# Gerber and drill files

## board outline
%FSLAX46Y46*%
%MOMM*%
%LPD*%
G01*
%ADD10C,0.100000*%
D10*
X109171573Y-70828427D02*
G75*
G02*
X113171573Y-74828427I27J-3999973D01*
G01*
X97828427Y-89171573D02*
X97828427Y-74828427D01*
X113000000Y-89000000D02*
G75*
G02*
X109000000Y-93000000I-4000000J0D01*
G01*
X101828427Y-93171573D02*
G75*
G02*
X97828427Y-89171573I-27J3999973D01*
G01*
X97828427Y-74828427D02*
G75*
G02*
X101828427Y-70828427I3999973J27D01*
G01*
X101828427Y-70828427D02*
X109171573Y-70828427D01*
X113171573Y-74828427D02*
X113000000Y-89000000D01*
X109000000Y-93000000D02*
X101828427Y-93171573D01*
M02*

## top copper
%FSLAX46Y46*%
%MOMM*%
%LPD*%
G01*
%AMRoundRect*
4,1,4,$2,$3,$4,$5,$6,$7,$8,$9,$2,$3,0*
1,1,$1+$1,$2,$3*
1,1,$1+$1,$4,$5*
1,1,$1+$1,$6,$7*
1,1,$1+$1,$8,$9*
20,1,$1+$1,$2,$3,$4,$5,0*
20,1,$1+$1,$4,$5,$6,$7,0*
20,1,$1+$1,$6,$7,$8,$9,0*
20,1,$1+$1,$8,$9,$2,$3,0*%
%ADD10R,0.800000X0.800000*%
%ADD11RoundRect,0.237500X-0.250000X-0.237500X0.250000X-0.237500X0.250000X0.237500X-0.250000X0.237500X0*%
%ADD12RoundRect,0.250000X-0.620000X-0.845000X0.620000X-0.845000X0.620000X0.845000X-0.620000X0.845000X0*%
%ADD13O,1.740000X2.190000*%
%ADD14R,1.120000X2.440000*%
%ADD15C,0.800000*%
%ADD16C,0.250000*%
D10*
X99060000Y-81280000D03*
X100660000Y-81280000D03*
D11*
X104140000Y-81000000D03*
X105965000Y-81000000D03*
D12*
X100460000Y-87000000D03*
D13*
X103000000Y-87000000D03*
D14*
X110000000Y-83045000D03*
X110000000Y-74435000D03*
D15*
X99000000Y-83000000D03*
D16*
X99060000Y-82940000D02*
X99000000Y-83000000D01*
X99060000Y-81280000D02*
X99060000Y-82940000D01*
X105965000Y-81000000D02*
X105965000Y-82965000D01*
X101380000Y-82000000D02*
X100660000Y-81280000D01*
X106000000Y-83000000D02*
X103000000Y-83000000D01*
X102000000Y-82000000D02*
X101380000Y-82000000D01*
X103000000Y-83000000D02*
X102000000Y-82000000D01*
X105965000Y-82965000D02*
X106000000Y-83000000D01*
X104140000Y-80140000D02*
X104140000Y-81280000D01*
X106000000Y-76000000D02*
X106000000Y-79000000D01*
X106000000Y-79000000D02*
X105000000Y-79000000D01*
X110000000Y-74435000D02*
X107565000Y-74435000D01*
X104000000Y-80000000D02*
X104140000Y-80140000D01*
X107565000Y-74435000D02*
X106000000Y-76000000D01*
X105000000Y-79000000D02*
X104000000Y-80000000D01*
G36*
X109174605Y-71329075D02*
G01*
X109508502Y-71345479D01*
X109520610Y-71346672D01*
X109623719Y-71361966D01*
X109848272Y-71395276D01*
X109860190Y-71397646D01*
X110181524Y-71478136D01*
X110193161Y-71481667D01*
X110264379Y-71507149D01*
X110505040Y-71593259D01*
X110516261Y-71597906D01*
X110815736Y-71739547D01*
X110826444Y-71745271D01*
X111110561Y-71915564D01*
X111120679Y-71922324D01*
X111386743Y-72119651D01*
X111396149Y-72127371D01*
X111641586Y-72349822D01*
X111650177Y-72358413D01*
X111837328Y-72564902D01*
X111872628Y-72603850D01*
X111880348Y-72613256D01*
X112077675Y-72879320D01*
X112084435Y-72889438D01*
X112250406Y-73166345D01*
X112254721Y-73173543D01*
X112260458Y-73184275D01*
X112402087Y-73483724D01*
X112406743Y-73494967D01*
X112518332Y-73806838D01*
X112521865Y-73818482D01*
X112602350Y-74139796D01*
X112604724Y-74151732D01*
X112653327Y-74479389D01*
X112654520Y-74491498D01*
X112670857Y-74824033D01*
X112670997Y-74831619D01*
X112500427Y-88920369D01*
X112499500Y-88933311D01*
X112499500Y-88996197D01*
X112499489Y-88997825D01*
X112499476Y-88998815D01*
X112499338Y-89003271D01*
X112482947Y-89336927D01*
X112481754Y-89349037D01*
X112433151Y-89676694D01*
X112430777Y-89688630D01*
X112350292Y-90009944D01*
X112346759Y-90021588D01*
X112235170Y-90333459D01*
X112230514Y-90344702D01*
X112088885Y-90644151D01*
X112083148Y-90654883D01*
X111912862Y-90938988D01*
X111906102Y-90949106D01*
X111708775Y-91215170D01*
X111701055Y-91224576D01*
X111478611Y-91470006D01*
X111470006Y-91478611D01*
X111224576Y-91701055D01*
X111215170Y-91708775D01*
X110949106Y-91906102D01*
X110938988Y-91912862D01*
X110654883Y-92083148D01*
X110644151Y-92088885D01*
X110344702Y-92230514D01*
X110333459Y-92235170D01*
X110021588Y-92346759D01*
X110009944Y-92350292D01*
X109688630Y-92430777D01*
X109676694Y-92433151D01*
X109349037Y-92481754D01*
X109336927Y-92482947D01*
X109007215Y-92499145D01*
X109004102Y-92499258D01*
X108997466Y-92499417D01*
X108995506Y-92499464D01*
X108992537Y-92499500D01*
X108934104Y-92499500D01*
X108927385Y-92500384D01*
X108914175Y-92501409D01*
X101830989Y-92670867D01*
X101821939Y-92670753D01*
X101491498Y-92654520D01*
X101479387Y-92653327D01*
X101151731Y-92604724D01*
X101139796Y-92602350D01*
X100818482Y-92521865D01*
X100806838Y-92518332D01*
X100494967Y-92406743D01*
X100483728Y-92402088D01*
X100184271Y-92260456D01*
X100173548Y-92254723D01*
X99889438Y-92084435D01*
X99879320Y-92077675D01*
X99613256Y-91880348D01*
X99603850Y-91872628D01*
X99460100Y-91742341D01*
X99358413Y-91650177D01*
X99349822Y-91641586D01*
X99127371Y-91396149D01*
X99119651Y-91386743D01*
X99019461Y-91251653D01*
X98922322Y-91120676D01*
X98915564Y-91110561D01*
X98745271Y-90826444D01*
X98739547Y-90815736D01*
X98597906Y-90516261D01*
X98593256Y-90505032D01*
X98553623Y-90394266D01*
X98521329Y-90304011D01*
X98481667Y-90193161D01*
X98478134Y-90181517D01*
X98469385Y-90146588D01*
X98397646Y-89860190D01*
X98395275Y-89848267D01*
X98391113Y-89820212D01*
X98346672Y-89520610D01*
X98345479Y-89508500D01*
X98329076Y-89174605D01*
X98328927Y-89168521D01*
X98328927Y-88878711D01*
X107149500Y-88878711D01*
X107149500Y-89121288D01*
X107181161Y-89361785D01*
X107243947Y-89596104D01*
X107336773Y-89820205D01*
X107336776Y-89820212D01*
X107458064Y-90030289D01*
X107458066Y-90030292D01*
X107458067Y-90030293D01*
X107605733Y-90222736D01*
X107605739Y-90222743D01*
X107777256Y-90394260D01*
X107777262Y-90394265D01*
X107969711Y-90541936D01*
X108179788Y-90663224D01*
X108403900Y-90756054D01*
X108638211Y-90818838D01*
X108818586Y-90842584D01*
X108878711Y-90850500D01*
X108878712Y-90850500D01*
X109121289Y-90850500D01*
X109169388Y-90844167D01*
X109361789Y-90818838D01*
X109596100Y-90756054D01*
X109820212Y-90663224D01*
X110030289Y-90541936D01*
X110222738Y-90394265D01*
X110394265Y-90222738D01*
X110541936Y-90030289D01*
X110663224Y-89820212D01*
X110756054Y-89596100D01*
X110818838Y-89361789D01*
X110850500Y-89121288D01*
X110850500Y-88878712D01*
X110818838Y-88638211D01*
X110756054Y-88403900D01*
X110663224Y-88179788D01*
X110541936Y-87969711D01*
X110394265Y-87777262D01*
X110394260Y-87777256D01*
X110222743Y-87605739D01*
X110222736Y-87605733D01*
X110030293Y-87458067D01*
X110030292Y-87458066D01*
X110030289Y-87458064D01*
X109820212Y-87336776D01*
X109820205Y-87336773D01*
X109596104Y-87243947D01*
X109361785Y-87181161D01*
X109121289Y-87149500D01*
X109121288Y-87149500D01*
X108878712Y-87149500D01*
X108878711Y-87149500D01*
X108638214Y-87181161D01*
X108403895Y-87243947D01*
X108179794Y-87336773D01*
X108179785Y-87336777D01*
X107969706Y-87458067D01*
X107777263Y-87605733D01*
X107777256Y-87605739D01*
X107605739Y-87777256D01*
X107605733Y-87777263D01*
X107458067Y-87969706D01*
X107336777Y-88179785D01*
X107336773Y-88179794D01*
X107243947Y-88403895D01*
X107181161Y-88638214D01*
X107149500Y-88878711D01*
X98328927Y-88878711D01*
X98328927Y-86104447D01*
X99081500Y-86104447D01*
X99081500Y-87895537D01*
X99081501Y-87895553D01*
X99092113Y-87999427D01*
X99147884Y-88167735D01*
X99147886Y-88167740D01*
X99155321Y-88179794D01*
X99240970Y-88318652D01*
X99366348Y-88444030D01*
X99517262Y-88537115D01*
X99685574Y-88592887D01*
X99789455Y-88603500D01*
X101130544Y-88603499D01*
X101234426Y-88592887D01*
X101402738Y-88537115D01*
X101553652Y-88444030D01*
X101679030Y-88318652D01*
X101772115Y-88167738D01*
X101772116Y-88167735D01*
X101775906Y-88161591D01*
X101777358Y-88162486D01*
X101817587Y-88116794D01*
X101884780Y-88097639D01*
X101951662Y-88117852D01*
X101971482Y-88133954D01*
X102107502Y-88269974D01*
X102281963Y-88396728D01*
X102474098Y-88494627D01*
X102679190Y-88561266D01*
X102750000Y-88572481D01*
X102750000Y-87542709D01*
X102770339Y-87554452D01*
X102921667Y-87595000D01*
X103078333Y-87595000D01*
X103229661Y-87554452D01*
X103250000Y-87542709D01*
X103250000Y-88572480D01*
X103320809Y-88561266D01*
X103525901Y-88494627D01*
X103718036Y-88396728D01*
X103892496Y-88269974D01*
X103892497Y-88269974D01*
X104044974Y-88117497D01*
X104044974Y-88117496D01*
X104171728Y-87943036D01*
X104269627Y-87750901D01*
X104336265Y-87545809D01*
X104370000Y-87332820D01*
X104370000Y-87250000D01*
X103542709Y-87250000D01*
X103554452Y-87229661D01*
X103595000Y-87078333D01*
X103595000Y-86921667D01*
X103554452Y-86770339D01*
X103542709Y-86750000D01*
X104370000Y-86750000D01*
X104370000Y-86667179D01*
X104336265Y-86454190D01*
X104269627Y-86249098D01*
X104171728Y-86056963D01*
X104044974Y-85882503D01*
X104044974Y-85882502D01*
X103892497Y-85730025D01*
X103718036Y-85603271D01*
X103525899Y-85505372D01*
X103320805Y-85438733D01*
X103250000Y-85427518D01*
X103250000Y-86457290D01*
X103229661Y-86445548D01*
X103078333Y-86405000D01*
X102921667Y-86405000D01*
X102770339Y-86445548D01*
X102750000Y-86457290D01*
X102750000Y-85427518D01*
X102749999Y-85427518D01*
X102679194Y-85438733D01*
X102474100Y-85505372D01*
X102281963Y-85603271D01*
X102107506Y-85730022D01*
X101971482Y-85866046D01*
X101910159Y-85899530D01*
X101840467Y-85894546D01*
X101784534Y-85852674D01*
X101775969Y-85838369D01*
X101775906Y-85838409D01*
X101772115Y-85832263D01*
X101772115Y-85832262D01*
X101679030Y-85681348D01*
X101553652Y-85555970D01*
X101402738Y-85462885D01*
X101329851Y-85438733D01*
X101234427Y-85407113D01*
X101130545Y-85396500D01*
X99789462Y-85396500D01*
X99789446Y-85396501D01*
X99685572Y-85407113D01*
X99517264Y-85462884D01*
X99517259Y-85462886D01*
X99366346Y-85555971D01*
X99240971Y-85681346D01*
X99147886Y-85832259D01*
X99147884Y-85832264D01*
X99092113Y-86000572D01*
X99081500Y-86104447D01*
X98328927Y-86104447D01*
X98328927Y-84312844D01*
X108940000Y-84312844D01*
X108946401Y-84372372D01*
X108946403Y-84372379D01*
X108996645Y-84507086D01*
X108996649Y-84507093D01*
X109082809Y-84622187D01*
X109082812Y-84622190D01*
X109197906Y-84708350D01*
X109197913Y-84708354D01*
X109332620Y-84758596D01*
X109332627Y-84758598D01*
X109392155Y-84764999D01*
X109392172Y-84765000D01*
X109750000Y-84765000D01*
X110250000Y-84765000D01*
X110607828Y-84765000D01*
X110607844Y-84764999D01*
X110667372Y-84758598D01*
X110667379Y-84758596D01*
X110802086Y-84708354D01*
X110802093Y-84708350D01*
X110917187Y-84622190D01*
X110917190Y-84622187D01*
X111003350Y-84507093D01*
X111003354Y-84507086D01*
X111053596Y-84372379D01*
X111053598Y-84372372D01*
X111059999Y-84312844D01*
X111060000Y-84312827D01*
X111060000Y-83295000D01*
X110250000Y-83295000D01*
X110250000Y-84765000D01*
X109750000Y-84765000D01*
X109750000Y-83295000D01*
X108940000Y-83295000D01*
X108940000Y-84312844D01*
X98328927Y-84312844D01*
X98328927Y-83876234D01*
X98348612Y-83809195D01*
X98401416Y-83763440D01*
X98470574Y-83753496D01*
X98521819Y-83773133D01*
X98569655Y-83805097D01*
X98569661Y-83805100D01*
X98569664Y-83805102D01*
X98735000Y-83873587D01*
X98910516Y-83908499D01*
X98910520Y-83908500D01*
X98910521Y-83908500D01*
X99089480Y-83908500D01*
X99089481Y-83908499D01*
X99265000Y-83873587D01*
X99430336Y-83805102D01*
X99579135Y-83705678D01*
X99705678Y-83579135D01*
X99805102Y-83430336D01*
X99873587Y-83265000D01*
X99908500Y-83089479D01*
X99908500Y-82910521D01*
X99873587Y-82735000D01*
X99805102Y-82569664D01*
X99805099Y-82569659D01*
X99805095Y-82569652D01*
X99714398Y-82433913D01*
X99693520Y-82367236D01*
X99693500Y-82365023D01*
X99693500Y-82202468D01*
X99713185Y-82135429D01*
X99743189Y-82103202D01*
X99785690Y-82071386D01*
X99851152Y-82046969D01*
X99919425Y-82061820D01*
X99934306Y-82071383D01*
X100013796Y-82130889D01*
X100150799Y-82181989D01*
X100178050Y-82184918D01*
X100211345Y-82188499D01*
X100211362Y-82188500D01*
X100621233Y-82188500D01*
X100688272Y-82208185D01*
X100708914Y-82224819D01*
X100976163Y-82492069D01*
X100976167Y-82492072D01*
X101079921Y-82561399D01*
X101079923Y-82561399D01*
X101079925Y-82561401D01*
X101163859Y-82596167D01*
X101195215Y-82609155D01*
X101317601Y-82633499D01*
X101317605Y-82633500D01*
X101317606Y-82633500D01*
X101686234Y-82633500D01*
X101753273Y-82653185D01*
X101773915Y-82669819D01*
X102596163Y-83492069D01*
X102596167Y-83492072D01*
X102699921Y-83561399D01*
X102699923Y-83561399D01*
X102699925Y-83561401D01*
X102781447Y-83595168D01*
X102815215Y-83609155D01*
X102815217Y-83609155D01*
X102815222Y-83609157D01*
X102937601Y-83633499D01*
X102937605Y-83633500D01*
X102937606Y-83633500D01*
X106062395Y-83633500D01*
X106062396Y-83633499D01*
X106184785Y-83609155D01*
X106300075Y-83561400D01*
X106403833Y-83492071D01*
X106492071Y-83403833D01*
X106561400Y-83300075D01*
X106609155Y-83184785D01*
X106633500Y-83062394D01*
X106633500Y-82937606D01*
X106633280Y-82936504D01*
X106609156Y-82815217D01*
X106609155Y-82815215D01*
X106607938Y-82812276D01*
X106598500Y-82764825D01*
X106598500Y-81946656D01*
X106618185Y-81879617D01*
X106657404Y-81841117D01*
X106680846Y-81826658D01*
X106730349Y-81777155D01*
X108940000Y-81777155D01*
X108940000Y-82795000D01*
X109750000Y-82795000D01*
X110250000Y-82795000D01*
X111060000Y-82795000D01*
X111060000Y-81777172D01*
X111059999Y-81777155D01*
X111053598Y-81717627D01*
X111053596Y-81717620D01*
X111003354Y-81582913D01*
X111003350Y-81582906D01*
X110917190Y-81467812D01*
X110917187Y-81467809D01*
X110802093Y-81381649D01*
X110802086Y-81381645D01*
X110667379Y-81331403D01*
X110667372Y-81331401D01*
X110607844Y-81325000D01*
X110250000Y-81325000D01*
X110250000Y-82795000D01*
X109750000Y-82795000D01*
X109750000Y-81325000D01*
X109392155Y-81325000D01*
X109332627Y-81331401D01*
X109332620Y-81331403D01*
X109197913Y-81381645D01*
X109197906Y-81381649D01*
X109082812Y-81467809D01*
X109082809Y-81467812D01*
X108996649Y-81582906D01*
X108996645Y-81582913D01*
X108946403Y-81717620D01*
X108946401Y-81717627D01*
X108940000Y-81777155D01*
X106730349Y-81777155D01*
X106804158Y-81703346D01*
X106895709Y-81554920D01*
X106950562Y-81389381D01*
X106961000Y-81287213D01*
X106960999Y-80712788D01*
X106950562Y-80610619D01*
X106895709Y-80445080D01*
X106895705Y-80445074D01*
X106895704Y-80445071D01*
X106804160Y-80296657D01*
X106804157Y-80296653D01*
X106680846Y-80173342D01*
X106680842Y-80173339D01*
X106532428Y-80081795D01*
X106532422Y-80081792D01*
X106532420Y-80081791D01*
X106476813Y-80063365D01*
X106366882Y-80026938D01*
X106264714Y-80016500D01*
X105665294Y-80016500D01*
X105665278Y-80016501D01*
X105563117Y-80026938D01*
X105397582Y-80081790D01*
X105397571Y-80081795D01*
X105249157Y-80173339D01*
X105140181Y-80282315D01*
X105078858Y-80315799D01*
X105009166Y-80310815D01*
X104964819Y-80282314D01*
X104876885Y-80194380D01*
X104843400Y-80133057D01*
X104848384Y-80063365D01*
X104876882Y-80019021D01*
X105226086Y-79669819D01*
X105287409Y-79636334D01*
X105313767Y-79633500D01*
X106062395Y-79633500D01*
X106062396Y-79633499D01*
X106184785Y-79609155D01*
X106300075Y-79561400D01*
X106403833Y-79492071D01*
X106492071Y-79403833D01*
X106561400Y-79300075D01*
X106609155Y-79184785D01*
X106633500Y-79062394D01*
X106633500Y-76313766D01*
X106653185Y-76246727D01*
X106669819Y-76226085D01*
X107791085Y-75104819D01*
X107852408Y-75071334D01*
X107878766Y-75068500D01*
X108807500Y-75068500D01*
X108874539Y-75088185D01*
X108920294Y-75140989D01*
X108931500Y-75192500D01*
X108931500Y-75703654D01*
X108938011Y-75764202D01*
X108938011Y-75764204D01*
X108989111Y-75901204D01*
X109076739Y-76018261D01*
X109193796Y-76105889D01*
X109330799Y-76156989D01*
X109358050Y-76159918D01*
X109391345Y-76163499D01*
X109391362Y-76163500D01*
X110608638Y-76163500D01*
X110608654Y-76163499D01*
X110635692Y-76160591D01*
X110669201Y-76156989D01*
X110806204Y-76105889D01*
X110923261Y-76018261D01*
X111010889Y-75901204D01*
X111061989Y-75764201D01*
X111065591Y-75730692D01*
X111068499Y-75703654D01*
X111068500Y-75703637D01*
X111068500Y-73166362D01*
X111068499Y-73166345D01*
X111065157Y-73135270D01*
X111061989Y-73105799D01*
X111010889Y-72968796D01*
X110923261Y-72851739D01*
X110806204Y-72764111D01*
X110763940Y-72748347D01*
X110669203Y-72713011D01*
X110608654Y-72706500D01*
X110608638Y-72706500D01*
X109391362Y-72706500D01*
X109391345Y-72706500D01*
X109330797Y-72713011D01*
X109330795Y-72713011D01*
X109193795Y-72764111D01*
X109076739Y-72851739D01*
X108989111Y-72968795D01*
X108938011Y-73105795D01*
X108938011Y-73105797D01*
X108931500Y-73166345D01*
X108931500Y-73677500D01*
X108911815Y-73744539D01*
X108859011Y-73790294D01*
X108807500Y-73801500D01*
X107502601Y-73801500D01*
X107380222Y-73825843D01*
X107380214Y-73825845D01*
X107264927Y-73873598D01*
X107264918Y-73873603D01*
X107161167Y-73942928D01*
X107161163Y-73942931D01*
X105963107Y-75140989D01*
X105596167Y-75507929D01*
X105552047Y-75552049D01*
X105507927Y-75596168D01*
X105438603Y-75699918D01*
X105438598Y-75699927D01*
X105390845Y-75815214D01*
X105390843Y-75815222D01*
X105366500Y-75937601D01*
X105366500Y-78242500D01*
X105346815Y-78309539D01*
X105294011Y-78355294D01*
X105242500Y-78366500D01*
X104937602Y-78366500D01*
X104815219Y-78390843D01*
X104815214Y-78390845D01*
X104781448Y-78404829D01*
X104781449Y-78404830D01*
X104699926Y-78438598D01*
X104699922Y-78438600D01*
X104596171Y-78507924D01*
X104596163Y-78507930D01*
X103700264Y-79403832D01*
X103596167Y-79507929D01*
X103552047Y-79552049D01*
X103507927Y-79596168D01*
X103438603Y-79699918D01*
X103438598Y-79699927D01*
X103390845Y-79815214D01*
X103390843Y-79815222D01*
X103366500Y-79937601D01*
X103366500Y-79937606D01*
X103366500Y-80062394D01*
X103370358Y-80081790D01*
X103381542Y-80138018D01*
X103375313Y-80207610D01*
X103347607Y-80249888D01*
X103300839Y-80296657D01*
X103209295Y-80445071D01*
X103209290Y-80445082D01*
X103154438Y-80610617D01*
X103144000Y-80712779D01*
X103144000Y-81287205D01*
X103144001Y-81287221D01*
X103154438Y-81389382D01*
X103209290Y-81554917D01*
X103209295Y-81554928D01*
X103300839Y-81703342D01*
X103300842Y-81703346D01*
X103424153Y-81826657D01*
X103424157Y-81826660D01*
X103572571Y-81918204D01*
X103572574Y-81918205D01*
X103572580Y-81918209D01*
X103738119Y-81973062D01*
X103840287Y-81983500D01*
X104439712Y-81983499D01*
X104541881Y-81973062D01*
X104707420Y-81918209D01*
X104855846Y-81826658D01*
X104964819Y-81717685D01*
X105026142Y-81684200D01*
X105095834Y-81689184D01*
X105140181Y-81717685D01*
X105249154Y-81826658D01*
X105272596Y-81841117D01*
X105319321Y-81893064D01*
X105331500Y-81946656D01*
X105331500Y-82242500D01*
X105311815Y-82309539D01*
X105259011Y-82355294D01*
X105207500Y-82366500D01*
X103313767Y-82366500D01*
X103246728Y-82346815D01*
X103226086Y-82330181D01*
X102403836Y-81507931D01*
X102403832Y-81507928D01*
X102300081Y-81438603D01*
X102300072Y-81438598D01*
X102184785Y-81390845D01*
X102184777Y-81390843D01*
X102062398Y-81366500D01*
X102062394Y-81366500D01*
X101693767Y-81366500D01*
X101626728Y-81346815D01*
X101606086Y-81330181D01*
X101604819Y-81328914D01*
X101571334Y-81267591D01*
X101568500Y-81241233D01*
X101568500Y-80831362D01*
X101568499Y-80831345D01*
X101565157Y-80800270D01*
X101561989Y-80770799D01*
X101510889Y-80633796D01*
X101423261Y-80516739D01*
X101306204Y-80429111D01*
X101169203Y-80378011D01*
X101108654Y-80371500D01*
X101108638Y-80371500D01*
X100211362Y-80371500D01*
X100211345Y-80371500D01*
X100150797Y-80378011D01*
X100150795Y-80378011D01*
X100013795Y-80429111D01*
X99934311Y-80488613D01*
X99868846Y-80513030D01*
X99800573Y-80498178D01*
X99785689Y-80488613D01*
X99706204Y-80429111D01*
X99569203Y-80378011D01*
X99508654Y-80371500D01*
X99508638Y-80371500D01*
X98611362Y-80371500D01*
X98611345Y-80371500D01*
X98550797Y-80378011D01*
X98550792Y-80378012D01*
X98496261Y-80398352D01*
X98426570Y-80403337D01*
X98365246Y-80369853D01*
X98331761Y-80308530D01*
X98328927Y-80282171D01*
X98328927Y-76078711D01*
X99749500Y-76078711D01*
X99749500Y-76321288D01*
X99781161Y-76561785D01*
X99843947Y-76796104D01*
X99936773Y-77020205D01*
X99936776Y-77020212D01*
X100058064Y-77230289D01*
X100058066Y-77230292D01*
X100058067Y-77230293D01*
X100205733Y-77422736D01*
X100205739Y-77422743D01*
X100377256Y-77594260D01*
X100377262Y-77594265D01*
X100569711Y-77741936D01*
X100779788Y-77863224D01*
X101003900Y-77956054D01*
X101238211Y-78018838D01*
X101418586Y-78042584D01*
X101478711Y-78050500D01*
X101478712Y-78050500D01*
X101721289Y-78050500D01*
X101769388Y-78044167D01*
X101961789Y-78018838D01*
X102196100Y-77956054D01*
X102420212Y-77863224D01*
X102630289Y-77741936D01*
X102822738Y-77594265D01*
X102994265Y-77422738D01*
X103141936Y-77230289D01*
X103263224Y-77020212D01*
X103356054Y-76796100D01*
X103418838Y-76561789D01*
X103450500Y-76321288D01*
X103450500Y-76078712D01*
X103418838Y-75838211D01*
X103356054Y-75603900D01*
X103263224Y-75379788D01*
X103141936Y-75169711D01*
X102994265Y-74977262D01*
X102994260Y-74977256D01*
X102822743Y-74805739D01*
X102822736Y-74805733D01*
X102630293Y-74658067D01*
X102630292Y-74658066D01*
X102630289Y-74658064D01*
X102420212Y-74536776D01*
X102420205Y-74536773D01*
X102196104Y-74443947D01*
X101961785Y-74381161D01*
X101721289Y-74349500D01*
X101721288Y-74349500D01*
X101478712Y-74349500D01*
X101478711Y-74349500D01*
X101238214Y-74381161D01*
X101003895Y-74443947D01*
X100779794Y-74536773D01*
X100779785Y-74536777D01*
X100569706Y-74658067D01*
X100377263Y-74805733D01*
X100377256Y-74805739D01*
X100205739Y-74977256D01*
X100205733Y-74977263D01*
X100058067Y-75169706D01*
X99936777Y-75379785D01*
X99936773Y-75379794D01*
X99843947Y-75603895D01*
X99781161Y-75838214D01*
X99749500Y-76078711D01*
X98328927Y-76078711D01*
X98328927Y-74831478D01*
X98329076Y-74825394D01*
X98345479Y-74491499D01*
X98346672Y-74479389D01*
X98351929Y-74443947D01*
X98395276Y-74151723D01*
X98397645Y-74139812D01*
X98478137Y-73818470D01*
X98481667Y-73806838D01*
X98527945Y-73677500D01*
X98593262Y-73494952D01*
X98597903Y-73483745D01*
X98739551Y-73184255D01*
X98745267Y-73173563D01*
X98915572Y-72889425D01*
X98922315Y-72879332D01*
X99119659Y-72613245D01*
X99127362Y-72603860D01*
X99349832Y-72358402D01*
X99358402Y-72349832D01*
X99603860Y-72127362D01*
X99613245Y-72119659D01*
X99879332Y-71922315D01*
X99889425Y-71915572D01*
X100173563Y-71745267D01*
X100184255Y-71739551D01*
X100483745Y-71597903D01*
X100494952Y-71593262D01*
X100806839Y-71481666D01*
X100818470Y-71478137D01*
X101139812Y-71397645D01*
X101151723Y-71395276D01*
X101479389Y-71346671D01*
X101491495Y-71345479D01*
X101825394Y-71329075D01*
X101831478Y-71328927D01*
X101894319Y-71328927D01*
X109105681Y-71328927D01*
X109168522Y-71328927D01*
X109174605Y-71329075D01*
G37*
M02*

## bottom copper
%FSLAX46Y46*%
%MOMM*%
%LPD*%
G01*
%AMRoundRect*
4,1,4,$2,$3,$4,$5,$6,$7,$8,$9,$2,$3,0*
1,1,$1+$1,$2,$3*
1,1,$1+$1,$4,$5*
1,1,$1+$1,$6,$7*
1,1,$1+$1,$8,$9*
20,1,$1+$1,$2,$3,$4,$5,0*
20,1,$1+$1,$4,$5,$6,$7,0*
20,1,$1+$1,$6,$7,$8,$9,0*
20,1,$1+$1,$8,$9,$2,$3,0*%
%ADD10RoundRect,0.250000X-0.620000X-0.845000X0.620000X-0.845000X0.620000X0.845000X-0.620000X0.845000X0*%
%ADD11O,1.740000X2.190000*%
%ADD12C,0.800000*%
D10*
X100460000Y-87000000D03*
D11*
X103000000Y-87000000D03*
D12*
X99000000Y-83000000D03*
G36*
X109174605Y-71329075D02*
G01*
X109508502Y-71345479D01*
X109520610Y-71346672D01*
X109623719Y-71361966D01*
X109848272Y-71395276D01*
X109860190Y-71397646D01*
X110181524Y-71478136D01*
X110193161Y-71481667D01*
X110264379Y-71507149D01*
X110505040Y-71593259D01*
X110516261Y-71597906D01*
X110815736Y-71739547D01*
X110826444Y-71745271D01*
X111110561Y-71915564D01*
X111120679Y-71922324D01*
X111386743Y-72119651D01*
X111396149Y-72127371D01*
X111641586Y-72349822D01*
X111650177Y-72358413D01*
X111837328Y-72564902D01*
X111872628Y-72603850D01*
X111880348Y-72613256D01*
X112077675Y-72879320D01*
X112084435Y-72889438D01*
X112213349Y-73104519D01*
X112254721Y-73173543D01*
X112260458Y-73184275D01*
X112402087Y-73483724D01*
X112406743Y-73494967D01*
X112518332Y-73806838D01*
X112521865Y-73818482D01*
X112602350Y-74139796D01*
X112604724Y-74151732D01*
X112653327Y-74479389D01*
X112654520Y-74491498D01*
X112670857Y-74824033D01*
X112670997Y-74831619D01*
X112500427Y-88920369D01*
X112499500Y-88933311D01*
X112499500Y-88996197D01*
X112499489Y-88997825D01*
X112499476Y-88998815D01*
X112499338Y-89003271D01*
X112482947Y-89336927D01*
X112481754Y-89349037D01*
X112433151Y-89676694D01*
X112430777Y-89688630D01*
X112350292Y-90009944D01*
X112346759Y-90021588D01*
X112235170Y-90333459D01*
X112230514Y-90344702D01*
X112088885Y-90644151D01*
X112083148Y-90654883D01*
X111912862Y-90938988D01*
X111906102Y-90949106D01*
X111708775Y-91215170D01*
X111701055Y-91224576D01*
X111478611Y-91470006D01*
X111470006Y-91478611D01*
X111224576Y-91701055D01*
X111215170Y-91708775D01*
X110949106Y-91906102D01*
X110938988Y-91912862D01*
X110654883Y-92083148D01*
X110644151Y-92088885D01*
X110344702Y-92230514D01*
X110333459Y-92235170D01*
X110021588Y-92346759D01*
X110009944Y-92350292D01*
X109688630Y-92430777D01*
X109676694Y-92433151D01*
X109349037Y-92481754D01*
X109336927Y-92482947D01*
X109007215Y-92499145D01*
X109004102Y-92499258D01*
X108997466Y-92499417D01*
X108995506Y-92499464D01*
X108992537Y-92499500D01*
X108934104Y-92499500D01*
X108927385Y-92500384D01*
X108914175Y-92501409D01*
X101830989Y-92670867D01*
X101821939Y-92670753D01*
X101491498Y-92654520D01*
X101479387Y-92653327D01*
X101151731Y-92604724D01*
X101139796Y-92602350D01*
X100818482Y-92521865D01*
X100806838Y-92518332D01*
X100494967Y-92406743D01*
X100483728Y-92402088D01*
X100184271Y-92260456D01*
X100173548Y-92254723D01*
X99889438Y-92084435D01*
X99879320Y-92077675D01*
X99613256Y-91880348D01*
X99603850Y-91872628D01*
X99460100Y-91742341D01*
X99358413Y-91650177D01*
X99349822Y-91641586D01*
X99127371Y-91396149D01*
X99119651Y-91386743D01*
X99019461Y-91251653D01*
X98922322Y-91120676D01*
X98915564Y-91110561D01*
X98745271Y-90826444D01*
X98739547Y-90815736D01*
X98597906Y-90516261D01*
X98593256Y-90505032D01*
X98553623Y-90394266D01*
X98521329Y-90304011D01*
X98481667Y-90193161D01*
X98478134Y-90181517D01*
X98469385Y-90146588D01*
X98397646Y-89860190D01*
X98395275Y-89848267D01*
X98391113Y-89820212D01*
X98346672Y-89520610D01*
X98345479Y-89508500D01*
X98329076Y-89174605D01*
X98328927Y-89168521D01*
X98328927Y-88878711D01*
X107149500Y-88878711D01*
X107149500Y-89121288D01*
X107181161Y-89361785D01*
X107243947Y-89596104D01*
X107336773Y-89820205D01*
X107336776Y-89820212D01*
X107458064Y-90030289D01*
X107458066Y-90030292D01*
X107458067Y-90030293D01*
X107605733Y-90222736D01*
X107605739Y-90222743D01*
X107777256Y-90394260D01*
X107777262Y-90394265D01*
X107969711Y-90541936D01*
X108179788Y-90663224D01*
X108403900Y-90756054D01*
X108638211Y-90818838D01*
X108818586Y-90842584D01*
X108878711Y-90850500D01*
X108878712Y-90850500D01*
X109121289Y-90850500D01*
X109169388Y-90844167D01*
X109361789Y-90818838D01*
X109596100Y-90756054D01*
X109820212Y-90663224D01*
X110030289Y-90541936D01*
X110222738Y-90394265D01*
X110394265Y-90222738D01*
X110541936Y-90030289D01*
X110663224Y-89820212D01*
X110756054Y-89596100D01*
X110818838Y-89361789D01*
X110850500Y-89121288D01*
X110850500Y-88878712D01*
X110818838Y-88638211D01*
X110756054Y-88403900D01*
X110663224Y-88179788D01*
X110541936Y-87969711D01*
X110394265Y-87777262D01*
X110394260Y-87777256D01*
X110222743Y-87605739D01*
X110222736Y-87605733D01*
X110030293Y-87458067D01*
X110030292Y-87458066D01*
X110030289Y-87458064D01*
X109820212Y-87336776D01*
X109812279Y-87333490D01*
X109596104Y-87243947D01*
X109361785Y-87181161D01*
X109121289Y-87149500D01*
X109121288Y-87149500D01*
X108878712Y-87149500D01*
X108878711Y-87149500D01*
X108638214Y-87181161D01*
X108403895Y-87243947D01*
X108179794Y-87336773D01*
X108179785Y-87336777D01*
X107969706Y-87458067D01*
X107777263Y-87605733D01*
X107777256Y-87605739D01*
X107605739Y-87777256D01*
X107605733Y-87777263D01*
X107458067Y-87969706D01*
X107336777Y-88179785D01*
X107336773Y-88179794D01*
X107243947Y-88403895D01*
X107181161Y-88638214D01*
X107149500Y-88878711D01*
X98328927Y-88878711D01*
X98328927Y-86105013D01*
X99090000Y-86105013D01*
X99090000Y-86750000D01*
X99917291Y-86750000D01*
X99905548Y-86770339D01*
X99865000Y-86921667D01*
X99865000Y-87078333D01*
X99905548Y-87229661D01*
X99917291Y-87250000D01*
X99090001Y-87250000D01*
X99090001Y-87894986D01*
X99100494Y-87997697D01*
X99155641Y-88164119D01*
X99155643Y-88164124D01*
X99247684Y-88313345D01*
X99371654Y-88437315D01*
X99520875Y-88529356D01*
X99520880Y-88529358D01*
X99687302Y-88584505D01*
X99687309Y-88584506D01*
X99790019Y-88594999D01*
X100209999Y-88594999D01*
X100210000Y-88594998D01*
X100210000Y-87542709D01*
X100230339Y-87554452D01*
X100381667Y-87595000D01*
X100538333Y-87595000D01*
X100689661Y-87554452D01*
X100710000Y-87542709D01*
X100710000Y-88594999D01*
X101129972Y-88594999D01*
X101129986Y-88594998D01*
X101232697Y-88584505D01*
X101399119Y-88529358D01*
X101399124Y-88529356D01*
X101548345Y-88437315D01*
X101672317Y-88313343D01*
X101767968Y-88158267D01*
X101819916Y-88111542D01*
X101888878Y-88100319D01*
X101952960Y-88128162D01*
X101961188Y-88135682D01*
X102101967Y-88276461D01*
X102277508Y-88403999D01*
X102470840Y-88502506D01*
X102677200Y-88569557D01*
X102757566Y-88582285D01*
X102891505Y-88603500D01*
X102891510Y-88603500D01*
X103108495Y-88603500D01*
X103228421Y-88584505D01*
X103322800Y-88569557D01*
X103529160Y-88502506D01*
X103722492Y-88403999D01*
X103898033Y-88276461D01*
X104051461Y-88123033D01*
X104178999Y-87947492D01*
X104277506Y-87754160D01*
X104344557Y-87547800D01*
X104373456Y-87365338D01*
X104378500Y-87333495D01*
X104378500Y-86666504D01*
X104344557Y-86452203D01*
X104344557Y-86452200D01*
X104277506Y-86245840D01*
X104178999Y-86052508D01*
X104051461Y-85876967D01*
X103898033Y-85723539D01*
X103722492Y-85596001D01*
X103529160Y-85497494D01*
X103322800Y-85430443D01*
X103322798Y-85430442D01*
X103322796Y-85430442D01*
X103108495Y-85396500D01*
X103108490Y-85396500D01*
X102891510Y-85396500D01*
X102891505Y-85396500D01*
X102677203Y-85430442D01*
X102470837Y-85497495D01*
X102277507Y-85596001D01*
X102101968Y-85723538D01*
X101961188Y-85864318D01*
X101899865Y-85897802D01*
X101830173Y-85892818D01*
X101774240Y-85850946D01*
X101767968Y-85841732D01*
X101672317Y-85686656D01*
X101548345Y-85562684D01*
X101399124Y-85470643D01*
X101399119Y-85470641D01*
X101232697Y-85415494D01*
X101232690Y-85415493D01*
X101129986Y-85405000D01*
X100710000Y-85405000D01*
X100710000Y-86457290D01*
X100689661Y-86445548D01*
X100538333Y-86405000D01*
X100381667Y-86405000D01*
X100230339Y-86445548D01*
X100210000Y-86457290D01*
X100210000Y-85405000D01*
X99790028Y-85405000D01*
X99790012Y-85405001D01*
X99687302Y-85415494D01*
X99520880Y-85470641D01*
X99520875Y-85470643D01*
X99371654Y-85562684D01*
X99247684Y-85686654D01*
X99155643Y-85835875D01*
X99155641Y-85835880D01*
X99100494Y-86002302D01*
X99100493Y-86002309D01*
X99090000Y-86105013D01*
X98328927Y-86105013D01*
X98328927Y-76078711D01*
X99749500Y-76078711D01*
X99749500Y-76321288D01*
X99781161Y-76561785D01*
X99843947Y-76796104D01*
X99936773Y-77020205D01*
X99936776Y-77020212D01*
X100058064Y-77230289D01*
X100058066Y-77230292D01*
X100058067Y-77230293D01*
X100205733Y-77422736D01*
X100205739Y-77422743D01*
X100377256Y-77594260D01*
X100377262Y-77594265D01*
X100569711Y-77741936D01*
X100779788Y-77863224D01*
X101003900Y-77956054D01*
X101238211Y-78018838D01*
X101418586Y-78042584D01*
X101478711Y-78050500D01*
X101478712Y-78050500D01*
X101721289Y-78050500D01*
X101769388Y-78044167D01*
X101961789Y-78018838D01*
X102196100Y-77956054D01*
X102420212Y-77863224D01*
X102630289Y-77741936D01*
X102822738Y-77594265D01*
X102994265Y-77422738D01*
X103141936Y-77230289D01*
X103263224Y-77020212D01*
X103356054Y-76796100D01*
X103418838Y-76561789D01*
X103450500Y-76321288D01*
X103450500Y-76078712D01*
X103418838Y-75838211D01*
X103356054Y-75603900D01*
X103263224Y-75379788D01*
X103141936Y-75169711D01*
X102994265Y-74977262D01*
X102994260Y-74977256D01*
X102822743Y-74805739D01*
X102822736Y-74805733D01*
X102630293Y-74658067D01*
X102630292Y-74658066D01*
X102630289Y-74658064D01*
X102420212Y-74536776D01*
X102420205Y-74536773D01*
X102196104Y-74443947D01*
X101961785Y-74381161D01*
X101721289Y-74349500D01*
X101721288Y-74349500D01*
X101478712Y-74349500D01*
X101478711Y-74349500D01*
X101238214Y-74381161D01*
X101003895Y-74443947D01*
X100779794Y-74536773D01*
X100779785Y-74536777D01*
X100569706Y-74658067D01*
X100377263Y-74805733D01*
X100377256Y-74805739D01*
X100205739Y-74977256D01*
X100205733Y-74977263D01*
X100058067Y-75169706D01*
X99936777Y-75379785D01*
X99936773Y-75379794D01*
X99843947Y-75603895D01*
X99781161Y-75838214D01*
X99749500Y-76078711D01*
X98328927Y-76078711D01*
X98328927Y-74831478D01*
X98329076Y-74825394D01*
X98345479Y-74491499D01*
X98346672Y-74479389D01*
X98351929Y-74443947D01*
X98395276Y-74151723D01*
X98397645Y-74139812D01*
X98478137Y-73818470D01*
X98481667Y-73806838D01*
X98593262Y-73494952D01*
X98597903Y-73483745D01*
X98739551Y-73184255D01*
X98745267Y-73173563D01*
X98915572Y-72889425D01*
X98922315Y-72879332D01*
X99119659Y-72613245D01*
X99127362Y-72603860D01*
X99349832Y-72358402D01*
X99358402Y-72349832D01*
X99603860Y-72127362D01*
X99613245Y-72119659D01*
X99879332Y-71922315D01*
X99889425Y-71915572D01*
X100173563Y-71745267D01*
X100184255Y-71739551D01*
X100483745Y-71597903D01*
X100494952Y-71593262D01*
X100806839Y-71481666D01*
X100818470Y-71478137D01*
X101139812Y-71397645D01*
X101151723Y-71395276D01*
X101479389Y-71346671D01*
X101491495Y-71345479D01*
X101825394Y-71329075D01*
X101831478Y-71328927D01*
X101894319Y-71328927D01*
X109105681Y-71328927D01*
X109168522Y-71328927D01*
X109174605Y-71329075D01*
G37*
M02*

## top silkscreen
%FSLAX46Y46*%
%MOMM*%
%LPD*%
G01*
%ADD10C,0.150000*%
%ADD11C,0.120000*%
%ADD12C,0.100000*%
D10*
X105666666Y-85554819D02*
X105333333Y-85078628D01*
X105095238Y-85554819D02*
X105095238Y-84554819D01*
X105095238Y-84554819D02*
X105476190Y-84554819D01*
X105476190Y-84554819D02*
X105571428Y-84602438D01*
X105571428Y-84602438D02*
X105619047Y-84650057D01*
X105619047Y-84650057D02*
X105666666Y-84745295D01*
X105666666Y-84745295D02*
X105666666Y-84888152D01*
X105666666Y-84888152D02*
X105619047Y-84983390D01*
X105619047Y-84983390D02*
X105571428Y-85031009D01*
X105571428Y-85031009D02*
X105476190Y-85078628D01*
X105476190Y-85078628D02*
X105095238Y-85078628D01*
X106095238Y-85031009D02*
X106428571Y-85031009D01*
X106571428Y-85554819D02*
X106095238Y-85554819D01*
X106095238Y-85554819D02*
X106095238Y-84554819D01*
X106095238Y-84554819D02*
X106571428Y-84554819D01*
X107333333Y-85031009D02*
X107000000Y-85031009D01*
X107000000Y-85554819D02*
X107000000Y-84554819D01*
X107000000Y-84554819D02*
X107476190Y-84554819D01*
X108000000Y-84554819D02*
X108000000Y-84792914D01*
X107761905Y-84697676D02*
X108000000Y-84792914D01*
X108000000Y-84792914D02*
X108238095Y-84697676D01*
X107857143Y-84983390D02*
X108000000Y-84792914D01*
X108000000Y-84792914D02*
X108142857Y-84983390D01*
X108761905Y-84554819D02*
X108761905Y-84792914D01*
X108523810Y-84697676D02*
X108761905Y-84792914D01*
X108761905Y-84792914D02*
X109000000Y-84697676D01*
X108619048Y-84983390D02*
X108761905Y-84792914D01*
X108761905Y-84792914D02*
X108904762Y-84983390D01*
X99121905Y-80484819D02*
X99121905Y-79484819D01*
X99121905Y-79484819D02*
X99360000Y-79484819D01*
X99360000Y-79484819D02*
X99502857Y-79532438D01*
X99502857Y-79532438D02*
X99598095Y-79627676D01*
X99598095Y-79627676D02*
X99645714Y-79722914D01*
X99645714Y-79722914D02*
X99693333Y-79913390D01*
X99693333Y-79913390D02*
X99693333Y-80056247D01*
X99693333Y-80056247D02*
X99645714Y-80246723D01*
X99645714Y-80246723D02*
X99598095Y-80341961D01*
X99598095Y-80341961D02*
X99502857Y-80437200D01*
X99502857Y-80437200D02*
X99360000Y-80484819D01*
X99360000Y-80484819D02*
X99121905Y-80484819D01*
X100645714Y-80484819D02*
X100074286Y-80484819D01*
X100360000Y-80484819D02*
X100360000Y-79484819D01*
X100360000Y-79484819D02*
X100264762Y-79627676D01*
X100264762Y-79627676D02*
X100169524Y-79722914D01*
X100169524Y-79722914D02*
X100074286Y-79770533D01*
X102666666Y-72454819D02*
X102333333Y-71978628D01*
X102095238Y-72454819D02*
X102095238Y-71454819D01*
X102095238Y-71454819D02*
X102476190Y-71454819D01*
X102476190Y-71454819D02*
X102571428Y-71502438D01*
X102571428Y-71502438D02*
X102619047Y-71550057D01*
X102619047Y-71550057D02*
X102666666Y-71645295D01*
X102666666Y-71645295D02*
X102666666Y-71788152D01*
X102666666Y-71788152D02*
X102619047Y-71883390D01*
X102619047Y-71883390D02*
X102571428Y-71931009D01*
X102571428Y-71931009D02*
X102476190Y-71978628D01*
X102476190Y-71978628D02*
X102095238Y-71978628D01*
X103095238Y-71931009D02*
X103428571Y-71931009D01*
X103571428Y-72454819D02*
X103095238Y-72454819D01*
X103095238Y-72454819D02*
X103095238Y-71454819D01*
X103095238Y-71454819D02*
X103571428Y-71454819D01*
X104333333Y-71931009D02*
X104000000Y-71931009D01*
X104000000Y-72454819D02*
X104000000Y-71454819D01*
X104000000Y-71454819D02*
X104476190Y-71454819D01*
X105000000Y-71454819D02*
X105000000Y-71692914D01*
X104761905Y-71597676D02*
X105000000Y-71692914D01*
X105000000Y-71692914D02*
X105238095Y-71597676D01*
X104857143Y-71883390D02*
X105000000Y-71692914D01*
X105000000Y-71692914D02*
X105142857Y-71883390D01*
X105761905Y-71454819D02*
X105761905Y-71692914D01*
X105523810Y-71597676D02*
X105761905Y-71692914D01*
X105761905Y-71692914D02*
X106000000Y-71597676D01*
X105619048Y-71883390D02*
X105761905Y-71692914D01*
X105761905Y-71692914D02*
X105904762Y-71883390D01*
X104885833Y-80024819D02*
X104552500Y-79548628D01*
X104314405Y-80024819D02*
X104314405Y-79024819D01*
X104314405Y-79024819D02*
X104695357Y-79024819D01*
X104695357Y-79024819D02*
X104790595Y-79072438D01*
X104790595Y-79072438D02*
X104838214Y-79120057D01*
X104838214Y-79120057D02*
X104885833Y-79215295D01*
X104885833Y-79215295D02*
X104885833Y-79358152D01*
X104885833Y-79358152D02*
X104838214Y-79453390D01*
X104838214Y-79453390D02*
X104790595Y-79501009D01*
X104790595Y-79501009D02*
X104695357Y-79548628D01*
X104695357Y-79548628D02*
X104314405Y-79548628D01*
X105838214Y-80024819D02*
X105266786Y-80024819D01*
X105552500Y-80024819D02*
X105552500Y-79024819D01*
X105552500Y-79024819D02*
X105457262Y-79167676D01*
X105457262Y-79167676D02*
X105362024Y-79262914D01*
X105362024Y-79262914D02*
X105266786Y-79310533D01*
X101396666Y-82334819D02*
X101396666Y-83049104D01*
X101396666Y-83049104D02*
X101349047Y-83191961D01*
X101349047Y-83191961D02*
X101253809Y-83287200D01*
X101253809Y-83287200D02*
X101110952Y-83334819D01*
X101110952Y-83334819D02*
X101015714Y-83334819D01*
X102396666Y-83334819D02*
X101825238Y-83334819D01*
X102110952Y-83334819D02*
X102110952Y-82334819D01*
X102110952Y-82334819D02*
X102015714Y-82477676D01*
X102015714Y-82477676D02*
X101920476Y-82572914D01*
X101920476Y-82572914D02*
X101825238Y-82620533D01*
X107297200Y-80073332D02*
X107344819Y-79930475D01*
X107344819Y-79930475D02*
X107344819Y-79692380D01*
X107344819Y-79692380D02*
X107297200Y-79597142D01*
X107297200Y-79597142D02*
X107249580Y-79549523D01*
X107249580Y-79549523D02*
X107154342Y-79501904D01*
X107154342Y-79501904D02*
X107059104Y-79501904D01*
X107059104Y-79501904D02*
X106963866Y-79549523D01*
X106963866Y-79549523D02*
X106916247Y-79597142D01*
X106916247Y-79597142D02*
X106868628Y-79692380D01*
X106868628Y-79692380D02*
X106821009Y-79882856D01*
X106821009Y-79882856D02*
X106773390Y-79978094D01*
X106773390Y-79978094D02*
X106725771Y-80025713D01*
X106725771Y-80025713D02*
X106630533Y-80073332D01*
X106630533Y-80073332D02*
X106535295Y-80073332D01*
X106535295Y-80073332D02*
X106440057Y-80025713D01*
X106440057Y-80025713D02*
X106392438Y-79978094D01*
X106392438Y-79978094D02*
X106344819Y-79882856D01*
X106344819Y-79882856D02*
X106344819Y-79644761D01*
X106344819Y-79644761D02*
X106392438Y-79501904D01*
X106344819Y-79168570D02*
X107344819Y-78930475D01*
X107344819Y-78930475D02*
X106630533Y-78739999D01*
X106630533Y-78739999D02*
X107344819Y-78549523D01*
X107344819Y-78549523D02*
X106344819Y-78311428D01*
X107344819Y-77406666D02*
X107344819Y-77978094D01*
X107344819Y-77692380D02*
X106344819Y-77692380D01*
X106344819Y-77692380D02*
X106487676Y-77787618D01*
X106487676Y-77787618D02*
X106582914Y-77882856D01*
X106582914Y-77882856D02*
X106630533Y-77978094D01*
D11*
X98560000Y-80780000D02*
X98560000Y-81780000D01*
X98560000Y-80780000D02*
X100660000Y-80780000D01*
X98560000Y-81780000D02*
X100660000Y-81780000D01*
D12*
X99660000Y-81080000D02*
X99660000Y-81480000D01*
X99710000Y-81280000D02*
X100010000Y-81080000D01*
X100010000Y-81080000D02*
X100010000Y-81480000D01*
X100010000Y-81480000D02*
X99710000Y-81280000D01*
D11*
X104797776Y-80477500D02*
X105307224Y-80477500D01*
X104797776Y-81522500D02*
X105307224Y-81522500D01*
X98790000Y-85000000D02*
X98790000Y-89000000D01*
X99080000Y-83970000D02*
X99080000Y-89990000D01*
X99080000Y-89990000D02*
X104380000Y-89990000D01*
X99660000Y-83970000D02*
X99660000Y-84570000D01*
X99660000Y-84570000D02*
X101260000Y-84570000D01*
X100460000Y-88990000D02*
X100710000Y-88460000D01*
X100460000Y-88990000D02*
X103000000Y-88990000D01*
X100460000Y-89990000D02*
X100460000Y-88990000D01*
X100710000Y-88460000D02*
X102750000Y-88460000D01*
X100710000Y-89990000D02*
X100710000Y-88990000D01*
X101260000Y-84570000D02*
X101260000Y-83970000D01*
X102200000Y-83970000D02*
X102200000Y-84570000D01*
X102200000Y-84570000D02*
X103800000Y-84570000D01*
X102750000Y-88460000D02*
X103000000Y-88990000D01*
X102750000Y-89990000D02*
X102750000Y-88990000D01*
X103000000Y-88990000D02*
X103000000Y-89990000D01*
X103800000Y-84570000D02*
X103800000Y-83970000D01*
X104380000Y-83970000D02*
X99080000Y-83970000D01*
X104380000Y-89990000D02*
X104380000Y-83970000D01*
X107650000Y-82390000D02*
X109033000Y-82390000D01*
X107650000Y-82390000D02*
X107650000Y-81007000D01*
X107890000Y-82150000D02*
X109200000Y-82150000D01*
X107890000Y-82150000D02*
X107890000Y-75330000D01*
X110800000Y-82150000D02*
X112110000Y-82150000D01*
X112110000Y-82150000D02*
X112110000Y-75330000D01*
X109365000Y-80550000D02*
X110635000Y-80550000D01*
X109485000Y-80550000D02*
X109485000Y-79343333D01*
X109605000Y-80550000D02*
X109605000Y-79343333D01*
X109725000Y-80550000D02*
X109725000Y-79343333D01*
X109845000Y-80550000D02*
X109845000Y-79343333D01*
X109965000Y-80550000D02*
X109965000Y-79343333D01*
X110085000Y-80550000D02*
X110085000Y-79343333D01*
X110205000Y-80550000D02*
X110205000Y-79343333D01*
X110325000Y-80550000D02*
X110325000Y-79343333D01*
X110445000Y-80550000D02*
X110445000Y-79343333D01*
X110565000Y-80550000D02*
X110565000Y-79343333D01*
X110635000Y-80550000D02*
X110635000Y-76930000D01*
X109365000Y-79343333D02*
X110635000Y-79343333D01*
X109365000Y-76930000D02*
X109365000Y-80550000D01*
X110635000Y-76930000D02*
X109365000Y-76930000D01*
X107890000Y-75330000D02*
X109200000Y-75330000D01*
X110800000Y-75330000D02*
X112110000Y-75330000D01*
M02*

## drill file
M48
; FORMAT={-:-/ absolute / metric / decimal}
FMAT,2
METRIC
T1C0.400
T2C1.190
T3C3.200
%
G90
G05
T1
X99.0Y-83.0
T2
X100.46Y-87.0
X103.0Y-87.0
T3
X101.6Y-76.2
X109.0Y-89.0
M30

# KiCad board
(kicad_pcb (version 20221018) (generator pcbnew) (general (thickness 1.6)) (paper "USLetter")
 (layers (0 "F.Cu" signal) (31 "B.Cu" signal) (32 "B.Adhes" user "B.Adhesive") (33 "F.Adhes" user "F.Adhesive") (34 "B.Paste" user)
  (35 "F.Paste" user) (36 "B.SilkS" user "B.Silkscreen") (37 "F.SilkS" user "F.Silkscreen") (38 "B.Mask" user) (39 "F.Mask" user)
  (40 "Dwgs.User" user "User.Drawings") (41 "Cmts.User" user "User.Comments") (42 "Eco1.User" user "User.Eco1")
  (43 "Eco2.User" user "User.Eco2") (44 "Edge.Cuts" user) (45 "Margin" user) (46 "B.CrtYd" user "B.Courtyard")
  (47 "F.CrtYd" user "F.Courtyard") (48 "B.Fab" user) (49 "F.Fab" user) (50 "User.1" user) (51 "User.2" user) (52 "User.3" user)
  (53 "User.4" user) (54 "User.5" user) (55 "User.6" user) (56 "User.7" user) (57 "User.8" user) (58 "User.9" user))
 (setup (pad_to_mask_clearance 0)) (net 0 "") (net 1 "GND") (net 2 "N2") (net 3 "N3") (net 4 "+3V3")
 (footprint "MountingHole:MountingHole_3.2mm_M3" (layer "F.Cu") (at 109 89)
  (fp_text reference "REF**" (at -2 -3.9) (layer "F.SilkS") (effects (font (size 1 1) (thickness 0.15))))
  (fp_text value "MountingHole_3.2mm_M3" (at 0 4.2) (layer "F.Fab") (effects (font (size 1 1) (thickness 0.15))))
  (pad "" np_thru_hole circle (at 0 0) (size 3.2 3.2) (drill 3.2) (layers "F&B.Cu" "*.Mask")))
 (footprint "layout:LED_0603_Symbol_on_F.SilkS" (layer "F.Cu") (at 99.86 81.28)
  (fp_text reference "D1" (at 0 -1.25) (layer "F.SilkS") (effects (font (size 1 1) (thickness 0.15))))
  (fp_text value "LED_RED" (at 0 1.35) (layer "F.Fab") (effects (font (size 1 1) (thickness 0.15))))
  (fp_line (start -1.3 -0.5) (end -1.3 0.5) (stroke (width 0.12) (type solid)) (layer "F.SilkS"))
  (fp_line (start -1.3 -0.5) (end 0.8 -0.5) (stroke (width 0.12) (type solid)) (layer "F.SilkS"))
  (fp_line (start -1.3 0.5) (end 0.8 0.5) (stroke (width 0.12) (type solid)) (layer "F.SilkS"))
  (fp_line (start -0.2 -0.2) (end -0.2 0.2) (stroke (width 0.1) (type solid)) (layer "F.SilkS"))
  (fp_line (start -0.15 0) (end 0.15 -0.2) (stroke (width 0.1) (type solid)) (layer "F.SilkS"))
  (fp_line (start 0.15 -0.2) (end 0.15 0.2) (stroke (width 0.1) (type solid)) (layer "F.SilkS"))
  (fp_line (start 0.15 0.2) (end -0.15 0) (stroke (width 0.1) (type solid)) (layer "F.SilkS"))
  (pad "1" smd rect (at -0.8 0 180) (size 0.8 0.8) (layers "F.Cu" "F.Paste" "F.Mask") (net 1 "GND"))
  (pad "2" smd rect (at 0.8 0 180) (size 0.8 0.8) (layers "F.Cu" "F.Paste" "F.Mask") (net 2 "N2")))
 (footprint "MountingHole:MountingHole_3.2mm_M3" (layer "F.Cu") (at 101.6 76.2)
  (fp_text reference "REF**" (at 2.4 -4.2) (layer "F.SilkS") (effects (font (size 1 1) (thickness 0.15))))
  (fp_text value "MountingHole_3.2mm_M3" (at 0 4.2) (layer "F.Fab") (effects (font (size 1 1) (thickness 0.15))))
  (pad "" np_thru_hole circle (at 0 0) (size 3.2 3.2) (drill 3.2) (layers "*.Cu" "*.Mask")))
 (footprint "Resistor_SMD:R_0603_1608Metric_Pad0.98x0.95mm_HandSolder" (layer "F.Cu") (at 105.0525 81)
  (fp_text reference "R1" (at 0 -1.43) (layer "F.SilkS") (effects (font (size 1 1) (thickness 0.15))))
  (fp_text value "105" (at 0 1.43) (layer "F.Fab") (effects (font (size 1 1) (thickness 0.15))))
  (fp_line (start -0.254724 -0.5225) (end 0.254724 -0.5225) (stroke (width 0.12) (type solid)) (layer "F.SilkS"))
  (fp_line (start -0.254724 0.5225) (end 0.254724 0.5225) (stroke (width 0.12) (type solid)) (layer "F.SilkS"))
  (pad "1" smd roundrect (at -0.9125 0) (size 0.975 0.95) (layers "F.Cu" "F.Paste" "F.Mask") (roundrect_rratio 0.25) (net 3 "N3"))
  (pad "2" smd roundrect (at 0.9125 0) (size 0.975 0.95) (layers "F.Cu" "F.Paste" "F.Mask") (roundrect_rratio 0.25) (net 2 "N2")))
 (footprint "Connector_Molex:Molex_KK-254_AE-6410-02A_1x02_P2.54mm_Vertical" (layer "F.Cu") (at 100.46 87)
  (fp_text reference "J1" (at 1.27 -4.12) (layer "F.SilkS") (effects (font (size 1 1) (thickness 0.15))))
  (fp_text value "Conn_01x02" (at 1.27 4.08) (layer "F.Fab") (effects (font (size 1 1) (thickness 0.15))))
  (fp_line (start -1.67 -2) (end -1.67 2) (stroke (width 0.12) (type solid)) (layer "F.SilkS"))
  (fp_line (start -1.38 -3.03) (end -1.38 2.99) (stroke (width 0.12) (type solid)) (layer "F.SilkS"))
  (fp_line (start -1.38 2.99) (end 3.92 2.99) (stroke (width 0.12) (type solid)) (layer "F.SilkS"))
  (fp_line (start -0.8 -3.03) (end -0.8 -2.43) (stroke (width 0.12) (type solid)) (layer "F.SilkS"))
  (fp_line (start -0.8 -2.43) (end 0.8 -2.43) (stroke (width 0.12) (type solid)) (layer "F.SilkS"))
  (fp_line (start 0 1.99) (end 0.25 1.46) (stroke (width 0.12) (type solid)) (layer "F.SilkS"))
  (fp_line (start 0 1.99) (end 2.54 1.99) (stroke (width 0.12) (type solid)) (layer "F.SilkS"))
  (fp_line (start 0 2.99) (end 0 1.99) (stroke (width 0.12) (type solid)) (layer "F.SilkS"))
  (fp_line (start 0.25 1.46) (end 2.29 1.46) (stroke (width 0.12) (type solid)) (layer "F.SilkS"))
  (fp_line (start 0.25 2.99) (end 0.25 1.99) (stroke (width 0.12) (type solid)) (layer "F.SilkS"))
  (fp_line (start 0.8 -2.43) (end 0.8 -3.03) (stroke (width 0.12) (type solid)) (layer "F.SilkS"))
  (fp_line (start 1.74 -3.03) (end 1.74 -2.43) (stroke (width 0.12) (type solid)) (layer "F.SilkS"))
  (fp_line (start 1.74 -2.43) (end 3.34 -2.43) (stroke (width 0.12) (type solid)) (layer "F.SilkS"))
  (fp_line (start 2.29 1.46) (end 2.54 1.99) (stroke (width 0.12) (type solid)) (layer "F.SilkS"))
  (fp_line (start 2.29 2.99) (end 2.29 1.99) (stroke (width 0.12) (type solid)) (layer "F.SilkS"))
  (fp_line (start 2.54 1.99) (end 2.54 2.99) (stroke (width 0.12) (type solid)) (layer "F.SilkS"))
  (fp_line (start 3.34 -2.43) (end 3.34 -3.03) (stroke (width 0.12) (type solid)) (layer "F.SilkS"))
  (fp_line (start 3.92 -3.03) (end -1.38 -3.03) (stroke (width 0.12) (type solid)) (layer "F.SilkS"))
  (fp_line (start 3.92 2.99) (end 3.92 -3.03) (stroke (width 0.12) (type solid)) (layer "F.SilkS"))
  (pad "1" thru_hole roundrect (at 0 0) (size 1.74 2.19) (drill 1.19) (layers "*.Cu" "*.Mask") (roundrect_rratio 0.143678) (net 1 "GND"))
  (pad "2" thru_hole oval (at 2.54 0) (size 1.74 2.19) (drill 1.19) (layers "*.Cu" "*.Mask") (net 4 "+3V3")))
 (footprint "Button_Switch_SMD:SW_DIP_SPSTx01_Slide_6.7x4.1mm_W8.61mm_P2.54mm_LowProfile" (layer "F.Cu") (at 110 78.74 90)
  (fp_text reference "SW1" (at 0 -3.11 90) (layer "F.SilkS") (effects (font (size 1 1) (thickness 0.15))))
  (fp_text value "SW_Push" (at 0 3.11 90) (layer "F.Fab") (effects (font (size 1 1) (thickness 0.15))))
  (fp_line (start -3.65 -2.35) (end -3.65 -0.967) (stroke (width 0.12) (type solid)) (layer "F.SilkS"))
  (fp_line (start -3.65 -2.35) (end -2.267 -2.35) (stroke (width 0.12) (type solid)) (layer "F.SilkS"))
  (fp_line (start -3.41 -2.11) (end -3.41 -0.8) (stroke (width 0.12) (type solid)) (layer "F.SilkS"))
  (fp_line (start -3.41 -2.11) (end 3.41 -2.11) (stroke (width 0.12) (type solid)) (layer "F.SilkS"))
  (fp_line (start -3.41 0.8) (end -3.41 2.11) (stroke (width 0.12) (type solid)) (layer "F.SilkS"))
  (fp_line (start -3.41 2.11) (end 3.41 2.11) (stroke (width 0.12) (type solid)) (layer "F.SilkS"))
  (fp_line (start -1.81 -0.635) (end -1.81 0.635) (stroke (width 0.12) (type solid)) (layer "F.SilkS"))
  (fp_line (start -1.81 -0.515) (end -0.603333 -0.515) (stroke (width 0.12) (type solid)) (layer "F.SilkS"))
  (fp_line (start -1.81 -0.395) (end -0.603333 -0.395) (stroke (width 0.12) (type solid)) (layer "F.SilkS"))
  (fp_line (start -1.81 -0.275) (end -0.603333 -0.275) (stroke (width 0.12) (type solid)) (layer "F.SilkS"))
  (fp_line (start -1.81 -0.155) (end -0.603333 -0.155) (stroke (width 0.12) (type solid)) (layer "F.SilkS"))
  (fp_line (start -1.81 -0.035) (end -0.603333 -0.035) (stroke (width 0.12) (type solid)) (layer "F.SilkS"))
  (fp_line (start -1.81 0.085) (end -0.603333 0.085) (stroke (width 0.12) (type solid)) (layer "F.SilkS"))
  (fp_line (start -1.81 0.205) (end -0.603333 0.205) (stroke (width 0.12) (type solid)) (layer "F.SilkS"))
  (fp_line (start -1.81 0.325) (end -0.603333 0.325) (stroke (width 0.12) (type solid)) (layer "F.SilkS"))
  (fp_line (start -1.81 0.445) (end -0.603333 0.445) (stroke (width 0.12) (type solid)) (layer "F.SilkS"))
  (fp_line (start -1.81 0.565) (end -0.603333 0.565) (stroke (width 0.12) (type solid)) (layer "F.SilkS"))
  (fp_line (start -1.81 0.635) (end 1.81 0.635) (stroke (width 0.12) (type solid)) (layer "F.SilkS"))
  (fp_line (start -0.603333 -0.635) (end -0.603333 0.635) (stroke (width 0.12) (type solid)) (layer "F.SilkS"))
  (fp_line (start 1.81 -0.635) (end -1.81 -0.635) (stroke (width 0.12) (type solid)) (layer "F.SilkS"))
  (fp_line (start 1.81 0.635) (end 1.81 -0.635) (stroke (width 0.12) (type solid)) (layer "F.SilkS"))
  (fp_line (start 3.41 -2.11) (end 3.41 -0.8) (stroke (width 0.12) (type solid)) (layer "F.SilkS"))
  (fp_line (start 3.41 0.8) (end 3.41 2.11) (stroke (width 0.12) (type solid)) (layer "F.SilkS"))
  (pad "1" smd rect (at -4.305 0 90) (size 2.44 1.12) (layers "F.Cu" "F.Paste" "F.Mask") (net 4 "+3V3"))
  (pad "2" smd rect (at 4.305 0 90) (size 2.44 1.12) (layers "F.Cu" "F.Paste" "F.Mask") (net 3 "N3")))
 (gr_arc (start 109.171573 70.828427) (mid 112 72) (end 113.171573 74.828427) (stroke (width 0.1) (type default)) (layer "Edge.Cuts"))
 (gr_line (start 97.828427 89.171573) (end 97.828427 74.828427) (stroke (width 0.1) (type default)) (layer "Edge.Cuts"))
 (gr_arc (start 113 89) (mid 111.828427 91.828427) (end 109 93) (stroke (width 0.1) (type default)) (layer "Edge.Cuts"))
 (gr_arc (start 101.828427 93.171573) (mid 99 92) (end 97.828427 89.171573) (stroke (width 0.1) (type default)) (layer "Edge.Cuts"))
 (gr_arc (start 97.828427 74.828427) (mid 99 72) (end 101.828427 70.828427) (stroke (width 0.1) (type default)) (layer "Edge.Cuts"))
 (gr_line (start 101.828427 70.828427) (end 109.171573 70.828427) (stroke (width 0.1) (type default)) (layer "Edge.Cuts"))
 (gr_line (start 113.171573 74.828427) (end 113 89) (stroke (width 0.1) (type default)) (layer "Edge.Cuts"))
 (gr_line (start 109 93) (end 101.828427 93.171573) (stroke (width 0.1) (type default)) (layer "Edge.Cuts"))
 (segment (start 99.06 82.94) (end 99 83) (width 0.25) (layer "F.Cu") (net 1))
 (segment (start 99.06 81.28) (end 99.06 82.94) (width 0.25) (layer "F.Cu") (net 1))
 (via (at 99 83) (size 0.8) (drill 0.4) (layers "F.Cu" "B.Cu") (free) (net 1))
 (segment (start 105.965 81) (end 105.965 82.965) (width 0.25) (layer "F.Cu") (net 2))
 (segment (start 101.38 82) (end 100.66 81.28) (width 0.25) (layer "F.Cu") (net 2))
 (segment (start 106 83) (end 103 83) (width 0.25) (layer "F.Cu") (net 2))
 (segment (start 102 82) (end 101.38 82) (width 0.25) (layer "F.Cu") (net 2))
 (segment (start 103 83) (end 102 82) (width 0.25) (layer "F.Cu") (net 2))
 (segment (start 105.965 82.965) (end 106 83) (width 0.25) (layer "F.Cu") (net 2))
 (segment (start 104.14 80.14) (end 104.14 81.28) (width 0.25) (layer "F.Cu") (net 3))
 (segment (start 106 76) (end 106 79) (width 0.25) (layer "F.Cu") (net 3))
 (segment (start 106 79) (end 105 79) (width 0.25) (layer "F.Cu") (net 3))
 (segment (start 110 74.435) (end 107.565 74.435) (width 0.25) (layer "F.Cu") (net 3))
 (segment (start 104 80) (end 104.14 80.14) (width 0.25) (layer "F.Cu") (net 3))
 (segment (start 107.565 74.435) (end 106 76) (width 0.25) (layer "F.Cu") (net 3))
 (segment (start 105 79) (end 104 80) (width 0.25) (layer "F.Cu") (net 3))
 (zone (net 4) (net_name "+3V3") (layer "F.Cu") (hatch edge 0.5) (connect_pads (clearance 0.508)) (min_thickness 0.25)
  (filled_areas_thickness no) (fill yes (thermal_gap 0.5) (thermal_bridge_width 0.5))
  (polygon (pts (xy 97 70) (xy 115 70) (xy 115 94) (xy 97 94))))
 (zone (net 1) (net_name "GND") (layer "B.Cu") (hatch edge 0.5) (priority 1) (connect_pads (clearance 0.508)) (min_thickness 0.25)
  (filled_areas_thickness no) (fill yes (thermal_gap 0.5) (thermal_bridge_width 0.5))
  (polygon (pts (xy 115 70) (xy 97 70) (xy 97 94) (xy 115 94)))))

